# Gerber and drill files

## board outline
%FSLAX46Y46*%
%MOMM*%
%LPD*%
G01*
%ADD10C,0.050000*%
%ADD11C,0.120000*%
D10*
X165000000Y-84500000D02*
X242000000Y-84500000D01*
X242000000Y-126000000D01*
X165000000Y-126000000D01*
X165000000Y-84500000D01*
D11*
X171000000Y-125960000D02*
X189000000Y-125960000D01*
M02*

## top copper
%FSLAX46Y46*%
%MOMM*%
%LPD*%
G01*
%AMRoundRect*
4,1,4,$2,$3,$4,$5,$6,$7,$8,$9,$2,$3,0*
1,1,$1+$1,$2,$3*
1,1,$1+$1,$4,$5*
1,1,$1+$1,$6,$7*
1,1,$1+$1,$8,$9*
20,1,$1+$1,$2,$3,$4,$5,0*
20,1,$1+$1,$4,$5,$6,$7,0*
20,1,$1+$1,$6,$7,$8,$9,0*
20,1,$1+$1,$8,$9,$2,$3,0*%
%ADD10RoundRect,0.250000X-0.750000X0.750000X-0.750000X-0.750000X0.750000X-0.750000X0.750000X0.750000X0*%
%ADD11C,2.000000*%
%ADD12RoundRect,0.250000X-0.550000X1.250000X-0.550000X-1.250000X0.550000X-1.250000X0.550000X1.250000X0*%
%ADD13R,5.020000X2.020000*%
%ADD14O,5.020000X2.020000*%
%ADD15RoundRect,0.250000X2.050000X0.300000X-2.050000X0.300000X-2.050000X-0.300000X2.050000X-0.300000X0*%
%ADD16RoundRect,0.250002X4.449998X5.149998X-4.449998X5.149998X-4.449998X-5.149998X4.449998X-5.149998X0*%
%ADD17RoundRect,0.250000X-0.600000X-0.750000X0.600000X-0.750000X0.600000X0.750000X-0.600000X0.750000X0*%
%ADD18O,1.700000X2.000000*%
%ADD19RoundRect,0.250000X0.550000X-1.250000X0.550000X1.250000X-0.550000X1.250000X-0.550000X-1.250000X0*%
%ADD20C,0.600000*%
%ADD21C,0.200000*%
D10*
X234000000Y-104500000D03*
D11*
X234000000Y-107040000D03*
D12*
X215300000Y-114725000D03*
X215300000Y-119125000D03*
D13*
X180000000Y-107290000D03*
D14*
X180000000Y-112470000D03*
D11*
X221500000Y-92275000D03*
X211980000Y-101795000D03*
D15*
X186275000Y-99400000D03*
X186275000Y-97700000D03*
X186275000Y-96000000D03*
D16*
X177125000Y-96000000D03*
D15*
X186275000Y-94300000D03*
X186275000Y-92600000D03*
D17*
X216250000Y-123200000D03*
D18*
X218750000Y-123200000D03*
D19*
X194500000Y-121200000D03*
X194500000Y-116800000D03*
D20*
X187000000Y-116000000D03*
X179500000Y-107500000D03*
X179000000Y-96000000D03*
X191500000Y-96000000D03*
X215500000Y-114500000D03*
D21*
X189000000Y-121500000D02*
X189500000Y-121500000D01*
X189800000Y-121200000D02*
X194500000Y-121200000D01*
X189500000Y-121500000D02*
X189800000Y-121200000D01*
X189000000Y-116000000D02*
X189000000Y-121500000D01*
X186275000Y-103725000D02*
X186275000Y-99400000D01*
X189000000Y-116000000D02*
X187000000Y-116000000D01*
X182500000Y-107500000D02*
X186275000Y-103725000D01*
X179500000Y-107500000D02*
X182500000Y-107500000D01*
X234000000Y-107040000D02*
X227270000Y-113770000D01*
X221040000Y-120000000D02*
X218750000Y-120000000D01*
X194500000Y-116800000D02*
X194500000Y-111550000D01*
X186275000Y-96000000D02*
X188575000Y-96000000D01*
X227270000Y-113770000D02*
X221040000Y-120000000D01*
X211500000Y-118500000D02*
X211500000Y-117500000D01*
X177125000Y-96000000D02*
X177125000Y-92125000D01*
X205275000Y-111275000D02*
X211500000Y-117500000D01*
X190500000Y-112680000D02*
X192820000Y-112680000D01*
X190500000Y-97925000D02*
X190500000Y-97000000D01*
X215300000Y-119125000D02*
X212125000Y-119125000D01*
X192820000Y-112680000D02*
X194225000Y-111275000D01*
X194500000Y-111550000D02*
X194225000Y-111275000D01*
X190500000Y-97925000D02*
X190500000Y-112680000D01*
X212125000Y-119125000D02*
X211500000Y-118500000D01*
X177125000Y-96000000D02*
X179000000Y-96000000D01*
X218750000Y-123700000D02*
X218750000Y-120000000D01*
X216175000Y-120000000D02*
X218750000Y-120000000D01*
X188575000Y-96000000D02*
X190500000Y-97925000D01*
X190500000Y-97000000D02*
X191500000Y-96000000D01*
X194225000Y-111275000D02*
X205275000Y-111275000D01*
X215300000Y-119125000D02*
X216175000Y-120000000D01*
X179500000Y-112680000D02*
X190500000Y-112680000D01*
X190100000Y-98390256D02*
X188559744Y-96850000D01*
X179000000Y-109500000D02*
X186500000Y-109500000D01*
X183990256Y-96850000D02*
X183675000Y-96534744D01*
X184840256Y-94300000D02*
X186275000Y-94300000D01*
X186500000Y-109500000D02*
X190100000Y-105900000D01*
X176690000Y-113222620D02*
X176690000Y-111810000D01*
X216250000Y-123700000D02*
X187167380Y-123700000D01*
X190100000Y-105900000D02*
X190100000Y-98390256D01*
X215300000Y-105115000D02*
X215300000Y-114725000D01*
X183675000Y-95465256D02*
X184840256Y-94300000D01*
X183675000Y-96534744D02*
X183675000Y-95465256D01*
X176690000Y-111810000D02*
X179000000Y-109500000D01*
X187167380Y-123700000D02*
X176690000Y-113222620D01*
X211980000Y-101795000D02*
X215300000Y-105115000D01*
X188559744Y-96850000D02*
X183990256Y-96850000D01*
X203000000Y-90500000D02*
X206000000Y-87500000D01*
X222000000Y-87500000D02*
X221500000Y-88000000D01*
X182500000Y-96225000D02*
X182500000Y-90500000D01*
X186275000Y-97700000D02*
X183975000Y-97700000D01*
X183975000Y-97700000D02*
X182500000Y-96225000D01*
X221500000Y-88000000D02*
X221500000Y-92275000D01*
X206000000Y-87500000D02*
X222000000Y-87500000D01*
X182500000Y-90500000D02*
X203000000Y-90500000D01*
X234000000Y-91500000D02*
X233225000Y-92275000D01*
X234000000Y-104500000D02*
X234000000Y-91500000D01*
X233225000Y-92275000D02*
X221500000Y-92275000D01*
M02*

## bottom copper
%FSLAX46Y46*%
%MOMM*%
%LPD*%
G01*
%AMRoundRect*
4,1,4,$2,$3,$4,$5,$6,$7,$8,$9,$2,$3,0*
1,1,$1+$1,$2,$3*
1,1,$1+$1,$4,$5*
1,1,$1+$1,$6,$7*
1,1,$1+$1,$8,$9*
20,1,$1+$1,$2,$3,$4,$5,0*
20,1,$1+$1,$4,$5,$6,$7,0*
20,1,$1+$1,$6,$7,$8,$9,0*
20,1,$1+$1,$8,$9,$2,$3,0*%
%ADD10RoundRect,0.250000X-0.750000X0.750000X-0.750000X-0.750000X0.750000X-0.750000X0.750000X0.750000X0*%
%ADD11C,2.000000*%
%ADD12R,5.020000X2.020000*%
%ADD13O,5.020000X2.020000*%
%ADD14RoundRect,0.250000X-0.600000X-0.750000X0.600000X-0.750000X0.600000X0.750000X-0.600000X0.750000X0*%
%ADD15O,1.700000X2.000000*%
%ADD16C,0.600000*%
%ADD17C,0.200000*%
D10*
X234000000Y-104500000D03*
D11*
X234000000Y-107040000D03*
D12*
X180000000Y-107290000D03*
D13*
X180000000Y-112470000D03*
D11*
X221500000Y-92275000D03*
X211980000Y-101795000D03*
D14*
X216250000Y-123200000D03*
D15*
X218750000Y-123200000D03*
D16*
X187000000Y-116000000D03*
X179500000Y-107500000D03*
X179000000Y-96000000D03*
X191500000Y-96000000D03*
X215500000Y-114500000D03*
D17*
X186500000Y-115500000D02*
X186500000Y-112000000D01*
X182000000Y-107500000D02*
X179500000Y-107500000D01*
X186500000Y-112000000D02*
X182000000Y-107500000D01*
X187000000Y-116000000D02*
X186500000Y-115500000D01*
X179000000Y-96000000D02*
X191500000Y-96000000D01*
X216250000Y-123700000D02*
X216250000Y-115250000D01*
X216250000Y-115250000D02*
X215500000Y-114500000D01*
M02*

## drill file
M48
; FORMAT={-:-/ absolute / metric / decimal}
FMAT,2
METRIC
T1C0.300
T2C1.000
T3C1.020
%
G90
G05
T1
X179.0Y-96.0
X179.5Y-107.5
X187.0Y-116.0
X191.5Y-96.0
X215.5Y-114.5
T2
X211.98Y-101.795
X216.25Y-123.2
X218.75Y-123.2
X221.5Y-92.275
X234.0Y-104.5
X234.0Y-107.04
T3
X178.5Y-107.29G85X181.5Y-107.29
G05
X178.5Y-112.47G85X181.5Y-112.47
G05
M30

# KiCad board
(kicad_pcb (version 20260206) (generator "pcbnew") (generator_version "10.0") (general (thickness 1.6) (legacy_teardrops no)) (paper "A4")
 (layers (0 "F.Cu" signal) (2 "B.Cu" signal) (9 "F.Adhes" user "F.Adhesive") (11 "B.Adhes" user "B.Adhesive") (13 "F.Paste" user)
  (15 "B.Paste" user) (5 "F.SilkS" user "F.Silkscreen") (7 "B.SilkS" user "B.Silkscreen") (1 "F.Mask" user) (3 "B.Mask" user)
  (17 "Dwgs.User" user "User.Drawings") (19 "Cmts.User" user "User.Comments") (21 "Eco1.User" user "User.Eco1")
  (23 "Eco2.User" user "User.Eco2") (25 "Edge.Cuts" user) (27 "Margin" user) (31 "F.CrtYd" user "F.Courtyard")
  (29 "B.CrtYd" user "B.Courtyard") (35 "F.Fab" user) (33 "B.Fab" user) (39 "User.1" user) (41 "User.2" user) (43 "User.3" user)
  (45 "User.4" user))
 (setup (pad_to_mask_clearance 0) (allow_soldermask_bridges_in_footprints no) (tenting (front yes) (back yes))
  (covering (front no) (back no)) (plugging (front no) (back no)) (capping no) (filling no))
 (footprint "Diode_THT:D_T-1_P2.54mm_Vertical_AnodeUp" (layer "F.Cu") (at 234 104.5 -90)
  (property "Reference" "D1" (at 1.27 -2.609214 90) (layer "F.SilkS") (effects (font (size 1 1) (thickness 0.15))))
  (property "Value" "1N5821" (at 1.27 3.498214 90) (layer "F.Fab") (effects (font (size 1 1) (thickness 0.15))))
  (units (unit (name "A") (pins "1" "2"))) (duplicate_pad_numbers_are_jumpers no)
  (pad "1" thru_hole roundrect (at 0 0 270) (size 2 2) (drill 1) (layers "*.Cu" "*.Mask") (remove_unused_layers no) (roundrect_rratio 0.125)
   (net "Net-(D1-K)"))
  (pad "2" thru_hole circle (at 2.54 0 270) (size 2 2) (drill 1) (layers "*.Cu" "*.Mask") (remove_unused_layers no) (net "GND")))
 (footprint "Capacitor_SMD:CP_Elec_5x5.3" (layer "F.Cu") (at 215.3 116.925 -90)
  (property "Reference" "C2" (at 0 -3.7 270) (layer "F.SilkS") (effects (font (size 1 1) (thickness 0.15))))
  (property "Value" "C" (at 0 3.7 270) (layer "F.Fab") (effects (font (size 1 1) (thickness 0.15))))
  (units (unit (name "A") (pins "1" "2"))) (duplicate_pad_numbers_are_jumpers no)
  (pad "1" smd roundrect (at -2.2 0 270) (size 3 1.6) (layers "F.Cu" "F.Mask" "F.Paste") (roundrect_rratio 0.15625) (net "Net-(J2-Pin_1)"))
  (pad "2" smd roundrect (at 2.2 0 270) (size 3 1.6) (layers "F.Cu" "F.Mask" "F.Paste") (roundrect_rratio 0.15625) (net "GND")))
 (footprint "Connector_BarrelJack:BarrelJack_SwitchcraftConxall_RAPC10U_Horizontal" (layer "F.Cu") (at 180 107.29 90)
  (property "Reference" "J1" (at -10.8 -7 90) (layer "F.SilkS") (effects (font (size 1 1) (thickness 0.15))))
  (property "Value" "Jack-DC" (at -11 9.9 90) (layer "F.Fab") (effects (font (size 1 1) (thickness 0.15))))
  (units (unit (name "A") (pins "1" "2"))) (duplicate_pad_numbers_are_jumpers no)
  (fp_line (start -18.67 -9) (end -18.67 9) (stroke (width 0.12) (type solid)) (layer "Edge.Cuts"))
  (pad "1" thru_hole rect (at 0 0 90) (size 2.02 5.02) (drill oval 1.02 4.02) (layers "*.Cu" "*.Mask") (remove_unused_layers no)
   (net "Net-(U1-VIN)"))
  (pad "2" thru_hole oval (at -5.18 0 90) (size 2.02 5.02) (drill oval 1.02 4.02) (layers "*.Cu" "*.Mask") (remove_unused_layers no)
   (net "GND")))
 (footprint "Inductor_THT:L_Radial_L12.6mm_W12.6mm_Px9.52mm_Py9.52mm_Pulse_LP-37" (layer "F.Cu") (at 221.5 92.275 180)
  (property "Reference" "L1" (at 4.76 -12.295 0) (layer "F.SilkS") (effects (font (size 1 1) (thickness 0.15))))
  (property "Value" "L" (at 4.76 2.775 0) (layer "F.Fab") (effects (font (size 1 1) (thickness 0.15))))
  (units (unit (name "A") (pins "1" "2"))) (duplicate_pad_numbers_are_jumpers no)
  (pad "1" thru_hole circle (at 0 0 180) (size 2 2) (drill 1) (layers "*.Cu" "*.Mask") (remove_unused_layers no) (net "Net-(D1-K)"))
  (pad "2" thru_hole circle (at 9.52 -9.52 180) (size 2 2) (drill 1) (layers "*.Cu" "*.Mask") (remove_unused_layers no)
   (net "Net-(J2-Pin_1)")))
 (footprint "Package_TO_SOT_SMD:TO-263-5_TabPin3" (layer "F.Cu") (at 178.625 96 180)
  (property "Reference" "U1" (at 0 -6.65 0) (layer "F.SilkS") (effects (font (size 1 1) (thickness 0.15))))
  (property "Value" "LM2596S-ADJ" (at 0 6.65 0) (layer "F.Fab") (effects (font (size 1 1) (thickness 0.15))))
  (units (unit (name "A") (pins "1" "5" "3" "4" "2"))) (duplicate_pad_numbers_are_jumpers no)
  (pad "" smd roundrect (at -0.925 -2.775 180) (size 4.55 5.25) (layers "F.Paste") (roundrect_rratio 0.054945))
  (pad "" smd roundrect (at -0.925 2.775 180) (size 4.55 5.25) (layers "F.Paste") (roundrect_rratio 0.054945))
  (pad "" smd roundrect (at 3.925 -2.775 180) (size 4.55 5.25) (layers "F.Paste") (roundrect_rratio 0.054945))
  (pad "" smd roundrect (at 3.925 2.775 180) (size 4.55 5.25) (layers "F.Paste") (roundrect_rratio 0.054945))
  (pad "1" smd roundrect (at -7.65 -3.4 180) (size 4.6 1.1) (layers "F.Cu" "F.Mask" "F.Paste") (roundrect_rratio 0.227273)
   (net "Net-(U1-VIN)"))
  (pad "2" smd roundrect (at -7.65 -1.7 180) (size 4.6 1.1) (layers "F.Cu" "F.Mask" "F.Paste") (roundrect_rratio 0.227273)
   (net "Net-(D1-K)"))
  (pad "3" smd roundrect (at -7.65 0 180) (size 4.6 1.1) (layers "F.Cu" "F.Mask" "F.Paste") (roundrect_rratio 0.227273) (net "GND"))
  (pad "3" smd roundrect (at 1.5 0 180) (size 9.4 10.8) (layers "F.Cu" "F.Mask") (roundrect_rratio 0.026596) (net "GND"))
  (pad "4" smd roundrect (at -7.65 1.7 180) (size 4.6 1.1) (layers "F.Cu" "F.Mask" "F.Paste") (roundrect_rratio 0.227273)
   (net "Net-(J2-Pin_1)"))
  (pad "5" smd roundrect (at -7.65 3.4 180) (size 4.6 1.1) (layers "F.Cu" "F.Mask" "F.Paste") (roundrect_rratio 0.227273)
   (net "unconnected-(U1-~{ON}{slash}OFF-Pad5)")))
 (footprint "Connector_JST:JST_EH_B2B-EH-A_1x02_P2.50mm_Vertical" (layer "F.Cu") (at 216.25 123.2)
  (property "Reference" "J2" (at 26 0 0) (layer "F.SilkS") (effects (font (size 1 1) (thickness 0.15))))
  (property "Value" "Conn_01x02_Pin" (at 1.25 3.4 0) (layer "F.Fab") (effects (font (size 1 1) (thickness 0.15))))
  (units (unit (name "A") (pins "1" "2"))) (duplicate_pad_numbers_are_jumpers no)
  (pad "1" thru_hole roundrect (at 0 0) (size 1.7 2) (drill 1) (layers "*.Cu" "*.Mask") (remove_unused_layers no)
   (roundrect_rratio 0.147059) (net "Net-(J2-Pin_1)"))
  (pad "2" thru_hole oval (at 2.5 0) (size 1.7 2) (drill 1) (layers "*.Cu" "*.Mask") (remove_unused_layers no) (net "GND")))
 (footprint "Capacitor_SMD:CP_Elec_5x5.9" (layer "F.Cu") (at 194.5 119 90)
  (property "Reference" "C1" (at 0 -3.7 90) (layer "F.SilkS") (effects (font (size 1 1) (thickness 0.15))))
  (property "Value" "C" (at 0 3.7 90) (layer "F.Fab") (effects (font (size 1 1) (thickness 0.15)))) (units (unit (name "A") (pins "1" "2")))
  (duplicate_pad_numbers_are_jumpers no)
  (pad "1" smd roundrect (at -2.2 0 90) (size 3 1.6) (layers "F.Cu" "F.Mask" "F.Paste") (roundrect_rratio 0.15625) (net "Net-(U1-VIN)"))
  (pad "2" smd roundrect (at 2.2 0 90) (size 3 1.6) (layers "F.Cu" "F.Mask" "F.Paste") (roundrect_rratio 0.15625) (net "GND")))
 (gr_rect (start 165 84.5) (end 242 126) (stroke (width 0.05) (type default)) (fill no) (layer "Edge.Cuts"))
 (segment (start 189 121.5) (end 189.5 121.5) (width 0.2) (layer "F.Cu") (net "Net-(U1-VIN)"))
 (segment (start 189.8 121.2) (end 194.5 121.2) (width 0.2) (layer "F.Cu") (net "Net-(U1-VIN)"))
 (segment (start 189.5 121.5) (end 189.8 121.2) (width 0.2) (layer "F.Cu") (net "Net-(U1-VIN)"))
 (segment (start 189 116) (end 189 121.5) (width 0.2) (layer "F.Cu") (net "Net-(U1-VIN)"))
 (segment (start 186.275 103.725) (end 186.275 99.4) (width 0.2) (layer "F.Cu") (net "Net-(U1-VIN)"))
 (segment (start 189 116) (end 187 116) (width 0.2) (layer "F.Cu") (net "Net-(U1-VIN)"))
 (segment (start 182.5 107.5) (end 186.275 103.725) (width 0.2) (layer "F.Cu") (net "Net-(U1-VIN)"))
 (segment (start 179.5 107.5) (end 182.5 107.5) (width 0.2) (layer "F.Cu") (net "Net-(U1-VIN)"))
 (via (at 187 116) (size 0.6) (drill 0.3) (layers "F.Cu" "B.Cu") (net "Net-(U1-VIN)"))
 (via (at 179.5 107.5) (size 0.6) (drill 0.3) (layers "F.Cu" "B.Cu") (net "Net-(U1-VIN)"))
 (segment (start 186.5 115.5) (end 186.5 112) (width 0.2) (layer "B.Cu") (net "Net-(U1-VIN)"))
 (segment (start 182 107.5) (end 179.5 107.5) (width 0.2) (layer "B.Cu") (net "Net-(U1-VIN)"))
 (segment (start 186.5 112) (end 182 107.5) (width 0.2) (layer "B.Cu") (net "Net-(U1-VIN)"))
 (segment (start 187 116) (end 186.5 115.5) (width 0.2) (layer "B.Cu") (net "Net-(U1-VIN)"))
 (segment (start 234 107.04) (end 227.27 113.77) (width 0.2) (layer "F.Cu") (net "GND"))
 (segment (start 221.04 120) (end 218.75 120) (width 0.2) (layer "F.Cu") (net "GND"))
 (segment (start 194.5 116.8) (end 194.5 111.55) (width 0.2) (layer "F.Cu") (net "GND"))
 (segment (start 186.275 96) (end 188.575 96) (width 0.2) (layer "F.Cu") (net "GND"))
 (segment (start 227.27 113.77) (end 221.04 120) (width 0.2) (layer "F.Cu") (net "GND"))
 (segment (start 211.5 118.5) (end 211.5 117.5) (width 0.2) (layer "F.Cu") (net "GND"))
 (segment (start 177.125 96) (end 177.125 92.125) (width 0.2) (layer "F.Cu") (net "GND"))
 (segment (start 205.275 111.275) (end 211.5 117.5) (width 0.2) (layer "F.Cu") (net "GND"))
 (segment (start 190.5 112.68) (end 192.82 112.68) (width 0.2) (layer "F.Cu") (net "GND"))
 (segment (start 190.5 97.925) (end 190.5 97) (width 0.2) (layer "F.Cu") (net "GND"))
 (segment (start 215.3 119.125) (end 212.125 119.125) (width 0.2) (layer "F.Cu") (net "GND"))
 (segment (start 192.82 112.68) (end 194.225 111.275) (width 0.2) (layer "F.Cu") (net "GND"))
 (segment (start 194.5 111.55) (end 194.225 111.275) (width 0.2) (layer "F.Cu") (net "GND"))
 (segment (start 190.5 97.925) (end 190.5 112.68) (width 0.2) (layer "F.Cu") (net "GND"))
 (segment (start 212.125 119.125) (end 211.5 118.5) (width 0.2) (layer "F.Cu") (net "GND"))
 (segment (start 177.125 96) (end 179 96) (width 0.2) (layer "F.Cu") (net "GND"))
 (segment (start 218.75 123.7) (end 218.75 120) (width 0.2) (layer "F.Cu") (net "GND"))
 (segment (start 216.175 120) (end 218.75 120) (width 0.2) (layer "F.Cu") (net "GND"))
 (segment (start 188.575 96) (end 190.5 97.925) (width 0.2) (layer "F.Cu") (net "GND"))
 (segment (start 190.5 97) (end 191.5 96) (width 0.2) (layer "F.Cu") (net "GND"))
 (segment (start 194.225 111.275) (end 205.275 111.275) (width 0.2) (layer "F.Cu") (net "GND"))
 (segment (start 215.3 119.125) (end 216.175 120) (width 0.2) (layer "F.Cu") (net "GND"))
 (segment (start 179.5 112.68) (end 190.5 112.68) (width 0.2) (layer "F.Cu") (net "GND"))
 (via (at 179 96) (size 0.6) (drill 0.3) (layers "F.Cu" "B.Cu") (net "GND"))
 (via (at 191.5 96) (size 0.6) (drill 0.3) (layers "F.Cu" "B.Cu") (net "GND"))
 (segment (start 179 96) (end 191.5 96) (width 0.2) (layer "B.Cu") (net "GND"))
 (segment (start 190.1 98.390256) (end 188.559744 96.85) (width 0.2) (layer "F.Cu") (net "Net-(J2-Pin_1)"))
 (segment (start 179 109.5) (end 186.5 109.5) (width 0.2) (layer "F.Cu") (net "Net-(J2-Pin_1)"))
 (segment (start 183.990256 96.85) (end 183.675 96.534744) (width 0.2) (layer "F.Cu") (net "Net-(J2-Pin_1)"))
 (segment (start 184.840256 94.3) (end 186.275 94.3) (width 0.2) (layer "F.Cu") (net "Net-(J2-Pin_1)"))
 (segment (start 186.5 109.5) (end 190.1 105.9) (width 0.2) (layer "F.Cu") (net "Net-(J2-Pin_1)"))
 (segment (start 176.69 113.22262) (end 176.69 111.81) (width 0.2) (layer "F.Cu") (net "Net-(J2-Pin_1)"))
 (segment (start 216.25 123.7) (end 187.16738 123.7) (width 0.2) (layer "F.Cu") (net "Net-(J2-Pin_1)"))
 (segment (start 190.1 105.9) (end 190.1 98.390256) (width 0.2) (layer "F.Cu") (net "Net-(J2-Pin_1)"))
 (segment (start 215.3 105.115) (end 215.3 114.725) (width 0.2) (layer "F.Cu") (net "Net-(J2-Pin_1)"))
 (segment (start 183.675 95.465256) (end 184.840256 94.3) (width 0.2) (layer "F.Cu") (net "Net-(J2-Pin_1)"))
 (segment (start 183.675 96.534744) (end 183.675 95.465256) (width 0.2) (layer "F.Cu") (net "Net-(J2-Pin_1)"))
 (segment (start 176.69 111.81) (end 179 109.5) (width 0.2) (layer "F.Cu") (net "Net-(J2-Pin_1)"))
 (segment (start 187.16738 123.7) (end 176.69 113.22262) (width 0.2) (layer "F.Cu") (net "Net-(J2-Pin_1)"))
 (segment (start 211.98 101.795) (end 215.3 105.115) (width 0.2) (layer "F.Cu") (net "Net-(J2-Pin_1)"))
 (segment (start 188.559744 96.85) (end 183.990256 96.85) (width 0.2) (layer "F.Cu") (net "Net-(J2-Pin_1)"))
 (via (at 215.5 114.5) (size 0.6) (drill 0.3) (layers "F.Cu" "B.Cu") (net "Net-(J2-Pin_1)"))
 (segment (start 216.25 123.7) (end 216.25 115.25) (width 0.2) (layer "B.Cu") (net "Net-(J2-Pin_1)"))
 (segment (start 216.25 115.25) (end 215.5 114.5) (width 0.2) (layer "B.Cu") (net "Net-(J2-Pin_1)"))
 (segment (start 203 90.5) (end 206 87.5) (width 0.2) (layer "F.Cu") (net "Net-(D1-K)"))
 (segment (start 222 87.5) (end 221.5 88) (width 0.2) (layer "F.Cu") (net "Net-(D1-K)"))
 (segment (start 182.5 96.225) (end 182.5 90.5) (width 0.2) (layer "F.Cu") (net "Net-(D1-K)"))
 (segment (start 186.275 97.7) (end 183.975 97.7) (width 0.2) (layer "F.Cu") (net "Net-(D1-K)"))
 (segment (start 183.975 97.7) (end 182.5 96.225) (width 0.2) (layer "F.Cu") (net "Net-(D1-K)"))
 (segment (start 221.5 88) (end 221.5 92.275) (width 0.2) (layer "F.Cu") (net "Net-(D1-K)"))
 (segment (start 206 87.5) (end 222 87.5) (width 0.2) (layer "F.Cu") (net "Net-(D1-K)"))
 (segment (start 182.5 90.5) (end 203 90.5) (width 0.2) (layer "F.Cu") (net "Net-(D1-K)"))
 (segment (start 234 91.5) (end 233.225 92.275) (width 0.2) (layer "F.Cu") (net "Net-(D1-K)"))
 (segment (start 234 104.5) (end 234 91.5) (width 0.2) (layer "F.Cu") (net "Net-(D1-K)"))
 (segment (start 233.225 92.275) (end 221.5 92.275) (width 0.2) (layer "F.Cu") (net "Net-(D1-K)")))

